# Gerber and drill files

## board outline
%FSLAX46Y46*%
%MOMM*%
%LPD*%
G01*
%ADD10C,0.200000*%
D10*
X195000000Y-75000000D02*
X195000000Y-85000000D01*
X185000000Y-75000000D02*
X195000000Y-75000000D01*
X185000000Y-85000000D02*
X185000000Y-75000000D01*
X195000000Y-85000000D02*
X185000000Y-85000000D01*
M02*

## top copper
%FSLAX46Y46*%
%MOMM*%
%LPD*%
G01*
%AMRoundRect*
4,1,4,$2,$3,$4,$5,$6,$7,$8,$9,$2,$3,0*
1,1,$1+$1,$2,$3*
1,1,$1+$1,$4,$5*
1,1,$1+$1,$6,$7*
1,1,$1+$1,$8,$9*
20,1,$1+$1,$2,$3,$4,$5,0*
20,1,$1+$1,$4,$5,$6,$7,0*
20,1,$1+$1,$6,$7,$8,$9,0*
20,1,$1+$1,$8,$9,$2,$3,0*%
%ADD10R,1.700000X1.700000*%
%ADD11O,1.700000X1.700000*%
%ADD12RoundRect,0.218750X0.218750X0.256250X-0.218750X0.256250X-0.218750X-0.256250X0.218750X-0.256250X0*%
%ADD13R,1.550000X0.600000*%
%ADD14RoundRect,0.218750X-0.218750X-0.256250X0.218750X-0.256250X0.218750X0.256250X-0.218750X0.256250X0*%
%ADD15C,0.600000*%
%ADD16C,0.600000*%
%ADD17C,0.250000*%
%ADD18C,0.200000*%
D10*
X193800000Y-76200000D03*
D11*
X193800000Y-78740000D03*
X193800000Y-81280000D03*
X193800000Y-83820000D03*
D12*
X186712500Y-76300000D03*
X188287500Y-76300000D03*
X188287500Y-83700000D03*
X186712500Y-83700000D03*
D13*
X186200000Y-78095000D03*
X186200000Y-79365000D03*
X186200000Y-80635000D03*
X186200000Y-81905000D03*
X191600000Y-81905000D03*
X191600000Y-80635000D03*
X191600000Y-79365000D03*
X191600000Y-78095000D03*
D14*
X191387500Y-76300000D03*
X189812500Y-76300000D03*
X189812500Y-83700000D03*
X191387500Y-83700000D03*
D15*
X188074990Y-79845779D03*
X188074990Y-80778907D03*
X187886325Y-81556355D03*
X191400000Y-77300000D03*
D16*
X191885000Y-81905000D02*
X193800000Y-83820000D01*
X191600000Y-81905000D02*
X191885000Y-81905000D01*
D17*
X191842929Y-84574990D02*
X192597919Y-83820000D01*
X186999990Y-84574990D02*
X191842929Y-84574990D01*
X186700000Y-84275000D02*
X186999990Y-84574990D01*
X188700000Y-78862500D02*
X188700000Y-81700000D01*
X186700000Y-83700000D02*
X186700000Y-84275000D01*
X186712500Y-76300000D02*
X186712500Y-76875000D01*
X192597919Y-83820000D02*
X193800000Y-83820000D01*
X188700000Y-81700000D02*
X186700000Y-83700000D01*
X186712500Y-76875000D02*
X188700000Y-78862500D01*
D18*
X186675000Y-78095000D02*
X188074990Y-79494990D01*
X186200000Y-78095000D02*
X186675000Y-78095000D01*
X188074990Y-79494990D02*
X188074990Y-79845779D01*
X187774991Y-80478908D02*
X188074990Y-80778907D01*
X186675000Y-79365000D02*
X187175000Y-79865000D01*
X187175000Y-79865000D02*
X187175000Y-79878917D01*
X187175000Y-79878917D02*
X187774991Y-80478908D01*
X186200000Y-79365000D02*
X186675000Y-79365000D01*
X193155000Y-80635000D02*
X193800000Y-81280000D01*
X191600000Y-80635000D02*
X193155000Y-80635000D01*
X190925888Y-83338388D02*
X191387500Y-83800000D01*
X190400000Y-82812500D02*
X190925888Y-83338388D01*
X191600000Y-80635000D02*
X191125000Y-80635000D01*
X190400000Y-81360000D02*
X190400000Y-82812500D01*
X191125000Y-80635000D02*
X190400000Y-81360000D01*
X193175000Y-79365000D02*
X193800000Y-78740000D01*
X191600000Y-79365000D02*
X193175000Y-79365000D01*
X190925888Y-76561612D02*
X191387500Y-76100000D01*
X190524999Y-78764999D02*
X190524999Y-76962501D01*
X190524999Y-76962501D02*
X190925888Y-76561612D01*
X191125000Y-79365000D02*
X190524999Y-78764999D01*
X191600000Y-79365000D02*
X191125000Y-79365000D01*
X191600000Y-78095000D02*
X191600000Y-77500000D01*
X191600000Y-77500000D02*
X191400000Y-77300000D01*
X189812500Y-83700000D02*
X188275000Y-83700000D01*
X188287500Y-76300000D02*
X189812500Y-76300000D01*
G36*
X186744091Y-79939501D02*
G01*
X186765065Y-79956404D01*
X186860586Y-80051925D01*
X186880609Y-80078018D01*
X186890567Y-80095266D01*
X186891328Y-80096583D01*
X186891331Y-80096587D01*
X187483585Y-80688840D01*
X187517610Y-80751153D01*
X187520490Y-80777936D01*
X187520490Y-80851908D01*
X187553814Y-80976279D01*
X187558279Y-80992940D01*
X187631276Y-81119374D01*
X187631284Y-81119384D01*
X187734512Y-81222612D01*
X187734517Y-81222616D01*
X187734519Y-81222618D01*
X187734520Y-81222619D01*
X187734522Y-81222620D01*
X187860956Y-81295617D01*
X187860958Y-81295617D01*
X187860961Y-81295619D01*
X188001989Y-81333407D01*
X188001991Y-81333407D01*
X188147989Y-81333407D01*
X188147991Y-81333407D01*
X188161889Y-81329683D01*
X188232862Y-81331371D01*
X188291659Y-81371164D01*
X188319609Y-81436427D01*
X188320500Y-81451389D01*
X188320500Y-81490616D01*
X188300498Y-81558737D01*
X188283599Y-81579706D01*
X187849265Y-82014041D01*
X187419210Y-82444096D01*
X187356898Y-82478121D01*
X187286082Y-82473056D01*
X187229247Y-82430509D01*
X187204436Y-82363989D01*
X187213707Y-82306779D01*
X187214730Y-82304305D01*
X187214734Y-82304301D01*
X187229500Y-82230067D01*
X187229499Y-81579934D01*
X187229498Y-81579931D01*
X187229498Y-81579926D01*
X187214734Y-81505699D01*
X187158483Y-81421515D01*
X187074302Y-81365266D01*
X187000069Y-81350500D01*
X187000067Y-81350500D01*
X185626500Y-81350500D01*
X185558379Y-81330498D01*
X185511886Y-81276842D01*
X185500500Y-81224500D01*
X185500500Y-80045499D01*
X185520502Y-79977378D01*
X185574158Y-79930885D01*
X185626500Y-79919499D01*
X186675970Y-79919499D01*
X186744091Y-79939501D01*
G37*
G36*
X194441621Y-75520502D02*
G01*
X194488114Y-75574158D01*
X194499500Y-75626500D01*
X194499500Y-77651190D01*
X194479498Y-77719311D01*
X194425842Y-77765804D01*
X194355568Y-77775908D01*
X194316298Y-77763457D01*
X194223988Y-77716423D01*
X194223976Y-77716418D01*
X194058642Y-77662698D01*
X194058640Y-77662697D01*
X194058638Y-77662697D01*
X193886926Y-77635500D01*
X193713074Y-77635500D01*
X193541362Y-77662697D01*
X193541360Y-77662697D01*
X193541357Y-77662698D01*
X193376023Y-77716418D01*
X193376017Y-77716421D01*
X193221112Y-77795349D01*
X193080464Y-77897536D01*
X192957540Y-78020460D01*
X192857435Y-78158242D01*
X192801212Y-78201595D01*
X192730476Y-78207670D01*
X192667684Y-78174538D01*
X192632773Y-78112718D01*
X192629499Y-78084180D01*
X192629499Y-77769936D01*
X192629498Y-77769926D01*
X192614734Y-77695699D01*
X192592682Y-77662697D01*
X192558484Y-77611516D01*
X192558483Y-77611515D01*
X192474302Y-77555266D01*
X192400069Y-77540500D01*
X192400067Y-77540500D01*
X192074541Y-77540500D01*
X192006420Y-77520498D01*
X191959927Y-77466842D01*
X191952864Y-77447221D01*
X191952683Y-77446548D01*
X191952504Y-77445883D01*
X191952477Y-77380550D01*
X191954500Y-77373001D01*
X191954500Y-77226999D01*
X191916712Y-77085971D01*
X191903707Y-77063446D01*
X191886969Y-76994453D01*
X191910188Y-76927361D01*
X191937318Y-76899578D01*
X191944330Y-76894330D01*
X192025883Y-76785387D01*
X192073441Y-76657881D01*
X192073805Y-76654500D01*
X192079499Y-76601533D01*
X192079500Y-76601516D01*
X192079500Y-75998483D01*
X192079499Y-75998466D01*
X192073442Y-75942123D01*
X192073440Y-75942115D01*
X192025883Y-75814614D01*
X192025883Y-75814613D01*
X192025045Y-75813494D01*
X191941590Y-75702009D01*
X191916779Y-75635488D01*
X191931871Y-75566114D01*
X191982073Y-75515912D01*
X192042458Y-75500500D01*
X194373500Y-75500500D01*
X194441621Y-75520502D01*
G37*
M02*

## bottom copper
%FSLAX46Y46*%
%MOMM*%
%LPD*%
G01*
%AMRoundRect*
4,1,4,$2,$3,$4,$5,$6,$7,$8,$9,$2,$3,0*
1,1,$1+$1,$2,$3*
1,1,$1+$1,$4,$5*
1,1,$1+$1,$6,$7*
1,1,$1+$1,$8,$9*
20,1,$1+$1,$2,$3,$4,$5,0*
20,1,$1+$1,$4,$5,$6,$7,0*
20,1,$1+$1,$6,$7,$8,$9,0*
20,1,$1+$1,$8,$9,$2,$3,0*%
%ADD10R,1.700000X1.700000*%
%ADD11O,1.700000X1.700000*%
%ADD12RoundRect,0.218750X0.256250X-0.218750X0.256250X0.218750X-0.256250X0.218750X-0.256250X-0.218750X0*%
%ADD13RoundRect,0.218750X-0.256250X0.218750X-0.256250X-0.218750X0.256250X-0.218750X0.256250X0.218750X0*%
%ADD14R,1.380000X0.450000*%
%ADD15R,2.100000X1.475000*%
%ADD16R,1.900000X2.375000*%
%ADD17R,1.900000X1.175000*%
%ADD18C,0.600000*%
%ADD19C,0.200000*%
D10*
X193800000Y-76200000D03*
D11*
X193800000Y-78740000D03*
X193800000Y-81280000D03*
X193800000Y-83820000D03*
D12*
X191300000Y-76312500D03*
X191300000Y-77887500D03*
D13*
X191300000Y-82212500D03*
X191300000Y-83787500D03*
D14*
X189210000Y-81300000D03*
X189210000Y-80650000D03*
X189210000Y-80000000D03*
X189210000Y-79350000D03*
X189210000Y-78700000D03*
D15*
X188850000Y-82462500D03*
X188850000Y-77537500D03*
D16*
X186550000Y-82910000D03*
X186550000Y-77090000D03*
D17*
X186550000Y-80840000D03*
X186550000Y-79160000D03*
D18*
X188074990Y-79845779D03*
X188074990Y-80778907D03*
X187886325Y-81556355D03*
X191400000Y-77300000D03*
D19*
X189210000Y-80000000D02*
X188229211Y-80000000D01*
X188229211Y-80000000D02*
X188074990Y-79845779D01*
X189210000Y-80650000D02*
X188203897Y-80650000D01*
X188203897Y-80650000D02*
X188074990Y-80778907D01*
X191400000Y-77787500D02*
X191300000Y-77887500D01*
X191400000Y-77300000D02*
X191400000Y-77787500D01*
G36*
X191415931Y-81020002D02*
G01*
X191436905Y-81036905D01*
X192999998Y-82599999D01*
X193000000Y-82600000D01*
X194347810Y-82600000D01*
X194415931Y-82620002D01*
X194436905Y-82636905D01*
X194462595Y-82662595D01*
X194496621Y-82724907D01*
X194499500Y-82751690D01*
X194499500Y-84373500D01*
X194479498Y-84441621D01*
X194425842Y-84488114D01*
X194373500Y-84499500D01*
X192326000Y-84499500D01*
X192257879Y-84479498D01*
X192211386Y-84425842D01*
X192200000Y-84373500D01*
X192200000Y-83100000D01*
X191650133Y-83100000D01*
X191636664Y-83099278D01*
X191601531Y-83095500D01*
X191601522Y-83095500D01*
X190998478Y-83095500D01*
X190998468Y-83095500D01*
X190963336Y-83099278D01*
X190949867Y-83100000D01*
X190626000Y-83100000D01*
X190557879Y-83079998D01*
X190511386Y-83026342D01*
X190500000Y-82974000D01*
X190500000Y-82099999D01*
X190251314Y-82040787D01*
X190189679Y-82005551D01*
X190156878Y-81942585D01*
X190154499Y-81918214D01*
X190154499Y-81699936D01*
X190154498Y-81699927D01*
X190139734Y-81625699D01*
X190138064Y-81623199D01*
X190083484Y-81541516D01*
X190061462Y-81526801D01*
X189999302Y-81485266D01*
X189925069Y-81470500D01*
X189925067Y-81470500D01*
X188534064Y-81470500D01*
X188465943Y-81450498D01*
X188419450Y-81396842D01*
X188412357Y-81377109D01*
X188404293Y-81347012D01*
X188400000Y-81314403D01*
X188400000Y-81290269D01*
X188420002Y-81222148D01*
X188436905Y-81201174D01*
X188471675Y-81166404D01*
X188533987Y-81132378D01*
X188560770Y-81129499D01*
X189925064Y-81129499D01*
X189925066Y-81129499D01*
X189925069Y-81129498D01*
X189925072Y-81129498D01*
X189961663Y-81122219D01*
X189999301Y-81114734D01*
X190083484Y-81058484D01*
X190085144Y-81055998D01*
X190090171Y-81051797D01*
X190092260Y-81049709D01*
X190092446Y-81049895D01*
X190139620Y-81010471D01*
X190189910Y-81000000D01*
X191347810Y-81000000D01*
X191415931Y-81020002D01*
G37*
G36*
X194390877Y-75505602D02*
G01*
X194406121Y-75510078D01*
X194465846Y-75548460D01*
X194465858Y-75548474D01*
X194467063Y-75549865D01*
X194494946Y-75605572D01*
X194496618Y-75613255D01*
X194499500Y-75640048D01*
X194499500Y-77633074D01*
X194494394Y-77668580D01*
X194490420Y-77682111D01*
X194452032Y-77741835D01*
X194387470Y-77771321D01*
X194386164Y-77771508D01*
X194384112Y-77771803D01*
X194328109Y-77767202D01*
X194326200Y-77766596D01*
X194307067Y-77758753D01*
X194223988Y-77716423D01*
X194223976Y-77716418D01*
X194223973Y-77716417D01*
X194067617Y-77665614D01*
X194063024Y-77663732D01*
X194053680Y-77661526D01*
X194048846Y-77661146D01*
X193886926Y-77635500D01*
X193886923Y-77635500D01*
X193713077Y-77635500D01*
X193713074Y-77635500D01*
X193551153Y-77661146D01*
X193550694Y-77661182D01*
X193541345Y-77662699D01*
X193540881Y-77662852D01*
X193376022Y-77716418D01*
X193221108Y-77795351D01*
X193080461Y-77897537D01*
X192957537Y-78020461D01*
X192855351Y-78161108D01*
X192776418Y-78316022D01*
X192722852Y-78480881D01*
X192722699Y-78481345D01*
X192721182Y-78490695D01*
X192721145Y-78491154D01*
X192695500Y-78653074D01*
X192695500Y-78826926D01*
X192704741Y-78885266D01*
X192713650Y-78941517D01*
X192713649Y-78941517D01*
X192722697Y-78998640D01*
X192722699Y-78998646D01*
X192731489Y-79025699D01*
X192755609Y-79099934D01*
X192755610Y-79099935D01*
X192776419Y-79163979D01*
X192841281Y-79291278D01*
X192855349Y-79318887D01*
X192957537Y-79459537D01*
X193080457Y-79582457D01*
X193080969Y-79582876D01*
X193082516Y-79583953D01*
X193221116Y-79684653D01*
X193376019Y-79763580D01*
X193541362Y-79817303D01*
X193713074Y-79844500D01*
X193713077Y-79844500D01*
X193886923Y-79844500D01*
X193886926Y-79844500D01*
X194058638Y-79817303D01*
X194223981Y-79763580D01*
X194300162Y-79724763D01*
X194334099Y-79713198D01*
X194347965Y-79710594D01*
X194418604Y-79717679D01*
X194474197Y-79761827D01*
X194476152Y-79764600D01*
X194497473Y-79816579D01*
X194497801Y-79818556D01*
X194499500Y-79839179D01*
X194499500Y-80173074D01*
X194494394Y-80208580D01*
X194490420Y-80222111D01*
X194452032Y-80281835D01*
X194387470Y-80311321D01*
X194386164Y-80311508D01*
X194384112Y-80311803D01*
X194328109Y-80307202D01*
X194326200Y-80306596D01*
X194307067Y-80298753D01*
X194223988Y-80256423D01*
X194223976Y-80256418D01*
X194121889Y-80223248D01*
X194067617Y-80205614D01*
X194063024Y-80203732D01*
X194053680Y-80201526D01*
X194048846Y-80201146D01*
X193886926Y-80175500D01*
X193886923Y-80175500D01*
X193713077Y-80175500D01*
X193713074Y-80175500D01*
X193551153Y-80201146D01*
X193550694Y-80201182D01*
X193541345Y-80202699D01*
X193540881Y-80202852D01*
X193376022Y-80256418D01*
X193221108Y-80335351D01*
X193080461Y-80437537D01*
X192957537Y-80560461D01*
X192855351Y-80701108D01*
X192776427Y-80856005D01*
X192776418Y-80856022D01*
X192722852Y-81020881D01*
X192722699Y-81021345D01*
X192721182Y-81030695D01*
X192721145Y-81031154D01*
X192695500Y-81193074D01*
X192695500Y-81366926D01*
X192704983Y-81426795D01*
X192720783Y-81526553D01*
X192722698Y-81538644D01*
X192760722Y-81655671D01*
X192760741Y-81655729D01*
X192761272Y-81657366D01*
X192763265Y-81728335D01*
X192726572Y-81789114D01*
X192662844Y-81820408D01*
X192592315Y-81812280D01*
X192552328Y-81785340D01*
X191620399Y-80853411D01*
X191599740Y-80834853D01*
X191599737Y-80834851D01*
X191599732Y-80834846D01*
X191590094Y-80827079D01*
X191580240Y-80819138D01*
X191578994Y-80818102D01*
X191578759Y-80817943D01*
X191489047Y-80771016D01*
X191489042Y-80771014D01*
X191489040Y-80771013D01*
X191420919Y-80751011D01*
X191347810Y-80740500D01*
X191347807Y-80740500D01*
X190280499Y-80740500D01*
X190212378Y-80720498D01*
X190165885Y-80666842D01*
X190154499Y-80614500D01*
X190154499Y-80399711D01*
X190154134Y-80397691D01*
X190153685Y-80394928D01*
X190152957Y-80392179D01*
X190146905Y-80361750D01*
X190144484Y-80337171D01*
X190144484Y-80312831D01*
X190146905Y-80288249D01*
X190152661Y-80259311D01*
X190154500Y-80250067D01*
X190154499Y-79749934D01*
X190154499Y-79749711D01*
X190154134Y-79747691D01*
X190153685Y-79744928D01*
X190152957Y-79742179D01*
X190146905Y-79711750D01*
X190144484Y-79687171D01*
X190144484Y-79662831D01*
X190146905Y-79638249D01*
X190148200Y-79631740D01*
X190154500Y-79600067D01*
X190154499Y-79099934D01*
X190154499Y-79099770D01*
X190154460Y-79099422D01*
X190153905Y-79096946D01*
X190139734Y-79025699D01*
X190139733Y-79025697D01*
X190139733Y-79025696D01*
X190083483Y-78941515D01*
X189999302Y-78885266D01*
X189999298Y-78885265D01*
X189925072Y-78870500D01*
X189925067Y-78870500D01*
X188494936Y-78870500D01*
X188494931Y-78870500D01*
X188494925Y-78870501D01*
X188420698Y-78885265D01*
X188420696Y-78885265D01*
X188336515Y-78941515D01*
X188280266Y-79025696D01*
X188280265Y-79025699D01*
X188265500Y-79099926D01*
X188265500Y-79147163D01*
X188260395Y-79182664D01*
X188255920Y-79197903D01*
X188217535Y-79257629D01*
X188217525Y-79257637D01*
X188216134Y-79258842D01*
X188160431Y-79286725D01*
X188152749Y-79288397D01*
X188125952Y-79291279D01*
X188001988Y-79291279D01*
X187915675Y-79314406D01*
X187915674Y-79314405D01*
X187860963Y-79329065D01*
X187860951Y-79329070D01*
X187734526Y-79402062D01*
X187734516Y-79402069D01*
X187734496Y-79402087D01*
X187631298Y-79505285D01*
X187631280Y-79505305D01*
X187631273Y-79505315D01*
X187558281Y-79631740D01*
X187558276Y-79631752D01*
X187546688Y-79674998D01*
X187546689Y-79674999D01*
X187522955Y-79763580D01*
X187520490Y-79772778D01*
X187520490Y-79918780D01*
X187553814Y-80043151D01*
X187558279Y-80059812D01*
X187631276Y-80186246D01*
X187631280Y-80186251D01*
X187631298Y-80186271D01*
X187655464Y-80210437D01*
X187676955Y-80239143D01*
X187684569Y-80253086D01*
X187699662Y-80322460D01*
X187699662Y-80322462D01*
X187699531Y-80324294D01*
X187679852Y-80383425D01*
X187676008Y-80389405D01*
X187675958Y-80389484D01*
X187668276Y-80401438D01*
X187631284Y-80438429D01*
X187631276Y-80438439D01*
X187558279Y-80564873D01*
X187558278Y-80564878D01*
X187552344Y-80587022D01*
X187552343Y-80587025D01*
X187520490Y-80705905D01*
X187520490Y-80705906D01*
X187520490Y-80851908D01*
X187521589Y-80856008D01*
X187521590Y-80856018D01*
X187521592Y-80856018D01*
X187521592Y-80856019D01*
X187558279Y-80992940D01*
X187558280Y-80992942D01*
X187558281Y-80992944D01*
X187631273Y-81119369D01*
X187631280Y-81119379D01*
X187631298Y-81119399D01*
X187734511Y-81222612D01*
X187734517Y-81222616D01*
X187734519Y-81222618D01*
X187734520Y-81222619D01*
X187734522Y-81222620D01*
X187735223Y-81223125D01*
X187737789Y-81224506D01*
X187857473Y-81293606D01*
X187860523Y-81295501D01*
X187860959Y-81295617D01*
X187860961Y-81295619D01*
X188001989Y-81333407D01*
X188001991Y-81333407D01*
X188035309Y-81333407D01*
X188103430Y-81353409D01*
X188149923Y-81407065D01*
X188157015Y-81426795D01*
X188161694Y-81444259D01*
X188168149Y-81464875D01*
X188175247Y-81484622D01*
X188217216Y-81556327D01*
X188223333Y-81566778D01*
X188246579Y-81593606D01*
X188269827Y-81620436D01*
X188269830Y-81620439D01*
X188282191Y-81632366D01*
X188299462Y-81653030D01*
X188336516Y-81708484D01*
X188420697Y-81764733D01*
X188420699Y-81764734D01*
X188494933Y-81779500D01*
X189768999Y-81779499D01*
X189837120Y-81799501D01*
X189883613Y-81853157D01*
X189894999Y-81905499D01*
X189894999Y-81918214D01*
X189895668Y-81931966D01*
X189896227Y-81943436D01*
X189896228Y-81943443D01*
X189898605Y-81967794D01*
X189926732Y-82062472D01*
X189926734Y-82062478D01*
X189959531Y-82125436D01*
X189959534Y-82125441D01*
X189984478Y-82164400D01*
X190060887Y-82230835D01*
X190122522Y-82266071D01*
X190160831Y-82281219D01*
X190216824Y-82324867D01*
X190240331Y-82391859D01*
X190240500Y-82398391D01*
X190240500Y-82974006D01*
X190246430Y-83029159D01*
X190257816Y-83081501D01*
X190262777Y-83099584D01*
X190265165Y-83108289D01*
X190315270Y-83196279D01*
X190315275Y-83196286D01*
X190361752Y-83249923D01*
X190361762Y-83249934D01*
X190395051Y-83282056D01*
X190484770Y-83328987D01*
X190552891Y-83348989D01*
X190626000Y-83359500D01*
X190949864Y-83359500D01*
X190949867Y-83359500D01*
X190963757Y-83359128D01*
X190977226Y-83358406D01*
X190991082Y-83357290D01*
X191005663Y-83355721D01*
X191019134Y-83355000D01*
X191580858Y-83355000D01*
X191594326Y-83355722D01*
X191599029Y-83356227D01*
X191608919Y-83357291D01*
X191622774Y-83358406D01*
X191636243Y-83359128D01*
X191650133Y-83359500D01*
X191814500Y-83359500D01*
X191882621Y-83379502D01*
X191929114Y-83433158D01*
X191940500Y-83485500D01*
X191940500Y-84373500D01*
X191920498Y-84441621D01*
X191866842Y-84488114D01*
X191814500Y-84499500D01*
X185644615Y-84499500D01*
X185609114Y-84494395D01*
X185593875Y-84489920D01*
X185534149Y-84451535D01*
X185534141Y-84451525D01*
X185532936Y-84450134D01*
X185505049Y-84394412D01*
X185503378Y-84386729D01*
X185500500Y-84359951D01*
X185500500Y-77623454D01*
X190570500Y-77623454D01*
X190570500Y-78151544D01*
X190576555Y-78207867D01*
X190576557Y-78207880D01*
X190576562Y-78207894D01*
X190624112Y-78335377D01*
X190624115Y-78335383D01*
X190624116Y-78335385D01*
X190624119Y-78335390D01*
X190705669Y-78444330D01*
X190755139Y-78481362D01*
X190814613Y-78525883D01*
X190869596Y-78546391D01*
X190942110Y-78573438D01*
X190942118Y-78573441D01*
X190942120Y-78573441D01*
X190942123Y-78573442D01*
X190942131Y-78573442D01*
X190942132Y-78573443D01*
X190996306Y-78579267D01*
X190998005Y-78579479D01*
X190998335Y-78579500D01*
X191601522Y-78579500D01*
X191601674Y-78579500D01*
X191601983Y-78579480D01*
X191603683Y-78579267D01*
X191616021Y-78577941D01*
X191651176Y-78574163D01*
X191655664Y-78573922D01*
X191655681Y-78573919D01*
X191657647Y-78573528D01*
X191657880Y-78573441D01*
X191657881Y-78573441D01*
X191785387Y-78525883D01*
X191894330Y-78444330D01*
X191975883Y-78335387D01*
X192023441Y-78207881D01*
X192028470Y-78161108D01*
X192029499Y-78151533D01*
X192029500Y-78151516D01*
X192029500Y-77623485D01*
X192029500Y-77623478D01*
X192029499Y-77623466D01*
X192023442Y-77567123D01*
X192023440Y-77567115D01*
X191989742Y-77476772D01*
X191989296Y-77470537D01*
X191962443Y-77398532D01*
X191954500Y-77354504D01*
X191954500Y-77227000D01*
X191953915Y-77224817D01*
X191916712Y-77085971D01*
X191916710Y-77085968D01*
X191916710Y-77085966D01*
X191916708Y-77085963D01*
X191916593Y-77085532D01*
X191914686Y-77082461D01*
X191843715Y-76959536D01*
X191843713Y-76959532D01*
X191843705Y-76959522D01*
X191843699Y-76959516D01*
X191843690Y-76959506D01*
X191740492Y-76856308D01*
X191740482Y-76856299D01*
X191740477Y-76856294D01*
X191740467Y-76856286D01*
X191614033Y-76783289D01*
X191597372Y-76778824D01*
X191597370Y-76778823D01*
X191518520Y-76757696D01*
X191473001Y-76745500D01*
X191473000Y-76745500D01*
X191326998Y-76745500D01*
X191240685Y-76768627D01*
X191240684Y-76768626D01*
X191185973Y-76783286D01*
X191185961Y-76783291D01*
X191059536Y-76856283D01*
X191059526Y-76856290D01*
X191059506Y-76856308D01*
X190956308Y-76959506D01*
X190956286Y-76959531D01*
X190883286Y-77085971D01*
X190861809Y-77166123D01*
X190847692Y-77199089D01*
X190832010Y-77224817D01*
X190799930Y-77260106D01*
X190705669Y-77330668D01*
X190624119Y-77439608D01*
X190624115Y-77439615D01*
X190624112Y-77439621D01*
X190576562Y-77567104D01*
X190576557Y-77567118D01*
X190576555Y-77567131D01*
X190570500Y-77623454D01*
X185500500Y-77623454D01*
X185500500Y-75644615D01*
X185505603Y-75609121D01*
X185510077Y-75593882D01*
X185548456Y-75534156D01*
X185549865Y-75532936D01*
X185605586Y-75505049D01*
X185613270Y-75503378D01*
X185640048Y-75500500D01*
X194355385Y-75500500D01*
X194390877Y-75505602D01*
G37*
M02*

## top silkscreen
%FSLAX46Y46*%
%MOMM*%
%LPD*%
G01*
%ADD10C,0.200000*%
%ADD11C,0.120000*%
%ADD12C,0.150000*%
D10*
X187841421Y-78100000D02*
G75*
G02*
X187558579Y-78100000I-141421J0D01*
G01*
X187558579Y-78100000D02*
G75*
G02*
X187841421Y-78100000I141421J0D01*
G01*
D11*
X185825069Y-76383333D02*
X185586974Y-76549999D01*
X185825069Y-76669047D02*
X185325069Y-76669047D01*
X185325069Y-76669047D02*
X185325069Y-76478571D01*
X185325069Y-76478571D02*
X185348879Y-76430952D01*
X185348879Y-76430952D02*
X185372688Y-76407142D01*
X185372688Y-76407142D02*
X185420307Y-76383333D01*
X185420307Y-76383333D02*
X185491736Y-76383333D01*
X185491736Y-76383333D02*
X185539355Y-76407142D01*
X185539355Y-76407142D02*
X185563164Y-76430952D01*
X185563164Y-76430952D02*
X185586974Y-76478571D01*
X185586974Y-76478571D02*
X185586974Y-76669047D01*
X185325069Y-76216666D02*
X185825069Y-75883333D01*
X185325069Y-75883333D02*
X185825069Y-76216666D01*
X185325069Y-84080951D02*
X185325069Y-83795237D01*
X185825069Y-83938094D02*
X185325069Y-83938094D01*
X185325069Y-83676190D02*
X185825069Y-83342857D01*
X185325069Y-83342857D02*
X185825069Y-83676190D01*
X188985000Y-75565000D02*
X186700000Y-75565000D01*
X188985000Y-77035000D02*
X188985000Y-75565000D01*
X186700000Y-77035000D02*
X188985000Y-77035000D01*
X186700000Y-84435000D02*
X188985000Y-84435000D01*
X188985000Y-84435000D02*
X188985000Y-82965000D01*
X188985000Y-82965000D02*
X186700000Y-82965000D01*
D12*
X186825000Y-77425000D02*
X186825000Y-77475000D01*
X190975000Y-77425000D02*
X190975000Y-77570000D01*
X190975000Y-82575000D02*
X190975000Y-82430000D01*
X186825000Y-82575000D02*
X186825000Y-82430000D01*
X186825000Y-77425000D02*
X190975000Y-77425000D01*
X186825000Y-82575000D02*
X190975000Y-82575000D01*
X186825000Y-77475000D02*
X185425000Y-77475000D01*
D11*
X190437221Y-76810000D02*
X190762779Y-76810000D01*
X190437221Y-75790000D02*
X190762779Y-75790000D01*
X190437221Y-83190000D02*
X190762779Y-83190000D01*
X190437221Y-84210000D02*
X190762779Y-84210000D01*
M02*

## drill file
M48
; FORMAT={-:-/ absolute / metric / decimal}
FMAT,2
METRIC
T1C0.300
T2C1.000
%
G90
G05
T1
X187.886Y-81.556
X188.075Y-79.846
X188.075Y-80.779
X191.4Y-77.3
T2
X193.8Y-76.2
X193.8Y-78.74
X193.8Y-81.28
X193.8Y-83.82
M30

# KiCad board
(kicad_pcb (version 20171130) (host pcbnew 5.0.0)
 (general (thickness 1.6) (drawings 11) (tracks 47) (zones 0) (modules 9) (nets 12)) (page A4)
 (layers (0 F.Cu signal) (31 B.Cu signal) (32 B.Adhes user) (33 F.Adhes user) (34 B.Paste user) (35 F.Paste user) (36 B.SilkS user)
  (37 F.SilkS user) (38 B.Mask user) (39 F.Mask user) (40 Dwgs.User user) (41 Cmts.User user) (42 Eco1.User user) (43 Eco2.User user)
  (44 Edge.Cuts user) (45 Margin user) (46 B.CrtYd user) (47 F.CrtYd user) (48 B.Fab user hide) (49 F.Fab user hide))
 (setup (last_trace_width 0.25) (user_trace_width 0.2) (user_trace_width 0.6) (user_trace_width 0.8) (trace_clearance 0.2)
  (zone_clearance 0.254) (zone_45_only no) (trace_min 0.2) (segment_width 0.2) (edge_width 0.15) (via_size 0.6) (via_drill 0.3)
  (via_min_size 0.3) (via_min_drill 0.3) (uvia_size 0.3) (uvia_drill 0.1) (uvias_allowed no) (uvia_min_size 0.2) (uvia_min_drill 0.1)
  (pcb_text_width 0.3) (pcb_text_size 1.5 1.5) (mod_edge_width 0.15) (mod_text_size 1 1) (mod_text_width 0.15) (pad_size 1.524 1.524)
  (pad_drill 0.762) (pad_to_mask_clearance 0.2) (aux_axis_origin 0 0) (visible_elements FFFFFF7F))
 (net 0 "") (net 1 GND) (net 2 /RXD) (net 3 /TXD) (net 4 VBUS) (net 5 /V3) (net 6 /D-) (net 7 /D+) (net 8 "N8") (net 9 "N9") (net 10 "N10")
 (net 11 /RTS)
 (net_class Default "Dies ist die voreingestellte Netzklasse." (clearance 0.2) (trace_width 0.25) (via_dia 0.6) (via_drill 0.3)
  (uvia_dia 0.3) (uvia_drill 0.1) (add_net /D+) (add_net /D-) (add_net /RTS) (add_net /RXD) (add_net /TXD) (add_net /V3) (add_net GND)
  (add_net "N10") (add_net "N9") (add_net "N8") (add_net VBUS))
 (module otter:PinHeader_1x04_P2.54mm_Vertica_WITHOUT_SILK (layer F.Cu) (at 193.8 76.2)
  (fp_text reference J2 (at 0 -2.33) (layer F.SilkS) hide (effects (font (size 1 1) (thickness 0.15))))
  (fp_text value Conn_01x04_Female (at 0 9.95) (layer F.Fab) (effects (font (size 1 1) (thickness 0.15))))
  (pad 1 thru_hole rect (at 0 0) (size 1.7 1.7) (drill 1) (layers *.Cu *.Mask) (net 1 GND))
  (pad 2 thru_hole oval (at 0 2.54) (size 1.7 1.7) (drill 1) (layers *.Cu *.Mask) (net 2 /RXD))
  (pad 3 thru_hole oval (at 0 5.08) (size 1.7 1.7) (drill 1) (layers *.Cu *.Mask) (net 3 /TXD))
  (pad 4 thru_hole oval (at 0 7.62) (size 1.7 1.7) (drill 1) (layers *.Cu *.Mask) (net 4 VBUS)))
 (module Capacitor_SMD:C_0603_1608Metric (layer B.Cu) (at 191.3 77.1 90)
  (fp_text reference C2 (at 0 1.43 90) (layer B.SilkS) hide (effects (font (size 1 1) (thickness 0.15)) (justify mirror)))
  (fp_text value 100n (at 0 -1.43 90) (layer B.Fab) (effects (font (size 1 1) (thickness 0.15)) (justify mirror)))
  (pad 2 smd roundrect (at 0.7875 0 90) (size 0.875 0.95) (layers B.Cu B.Paste B.Mask) (roundrect_rratio 0.25) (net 1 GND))
  (pad 1 smd roundrect (at -0.7875 0 90) (size 0.875 0.95) (layers B.Cu B.Paste B.Mask) (roundrect_rratio 0.25) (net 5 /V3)))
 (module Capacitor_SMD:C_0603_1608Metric (layer B.Cu) (at 191.3 83 270)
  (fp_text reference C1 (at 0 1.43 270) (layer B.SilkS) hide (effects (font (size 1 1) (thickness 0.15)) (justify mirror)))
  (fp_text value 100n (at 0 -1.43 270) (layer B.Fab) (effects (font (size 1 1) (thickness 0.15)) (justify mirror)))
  (pad 1 smd roundrect (at -0.7875 0 270) (size 0.875 0.95) (layers B.Cu B.Paste B.Mask) (roundrect_rratio 0.25) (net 4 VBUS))
  (pad 2 smd roundrect (at 0.7875 0 270) (size 0.875 0.95) (layers B.Cu B.Paste B.Mask) (roundrect_rratio 0.25) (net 1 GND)))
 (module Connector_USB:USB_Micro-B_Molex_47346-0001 (layer B.Cu) (at 187.75 80 90)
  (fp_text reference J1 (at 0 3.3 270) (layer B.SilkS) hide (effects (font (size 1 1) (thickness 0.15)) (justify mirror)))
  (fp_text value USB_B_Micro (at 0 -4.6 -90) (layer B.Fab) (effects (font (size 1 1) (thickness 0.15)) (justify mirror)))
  (pad 1 smd rect (at -1.3 1.46 90) (size 0.45 1.38) (layers B.Cu B.Paste B.Mask) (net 4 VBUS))
  (pad 2 smd rect (at -0.65 1.46 90) (size 0.45 1.38) (layers B.Cu B.Paste B.Mask) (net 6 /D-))
  (pad 3 smd rect (at 0 1.46 90) (size 0.45 1.38) (layers B.Cu B.Paste B.Mask) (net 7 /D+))
  (pad 4 smd rect (at 0.65 1.46 90) (size 0.45 1.38) (layers B.Cu B.Paste B.Mask) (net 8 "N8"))
  (pad 5 smd rect (at 1.3 1.46 90) (size 0.45 1.38) (layers B.Cu B.Paste B.Mask) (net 1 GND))
  (pad 6 smd rect (at -2.4625 1.1 90) (size 1.475 2.1) (layers B.Cu B.Paste B.Mask) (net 1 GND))
  (pad 6 smd rect (at 2.4625 1.1 90) (size 1.475 2.1) (layers B.Cu B.Paste B.Mask) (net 1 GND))
  (pad 6 smd rect (at -2.91 -1.2 90) (size 2.375 1.9) (layers B.Cu B.Paste B.Mask) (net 1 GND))
  (pad 6 smd rect (at 2.91 -1.2 90) (size 2.375 1.9) (layers B.Cu B.Paste B.Mask) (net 1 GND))
  (pad 6 smd rect (at -0.84 -1.2 90) (size 1.175 1.9) (layers B.Cu B.Paste B.Mask) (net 1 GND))
  (pad 6 smd rect (at 0.84 -1.2 90) (size 1.175 1.9) (layers B.Cu B.Paste B.Mask) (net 1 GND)))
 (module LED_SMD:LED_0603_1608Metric (layer F.Cu) (at 187.5 76.3 180)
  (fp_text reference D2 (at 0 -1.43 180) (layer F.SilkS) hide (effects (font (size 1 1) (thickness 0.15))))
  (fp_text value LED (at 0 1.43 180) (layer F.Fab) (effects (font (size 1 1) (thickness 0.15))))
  (fp_line (start -1.485 0.735) (end 0.8 0.735) (layer F.SilkS) (width 0.12))
  (fp_line (start -1.485 -0.735) (end -1.485 0.735) (layer F.SilkS) (width 0.12))
  (fp_line (start 0.8 -0.735) (end -1.485 -0.735) (layer F.SilkS) (width 0.12))
  (pad 2 smd roundrect (at 0.7875 0 180) (size 0.875 0.95) (layers F.Cu F.Paste F.Mask) (roundrect_rratio 0.25) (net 4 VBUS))
  (pad 1 smd roundrect (at -0.7875 0 180) (size 0.875 0.95) (layers F.Cu F.Paste F.Mask) (roundrect_rratio 0.25) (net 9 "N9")))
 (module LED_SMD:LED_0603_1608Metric (layer F.Cu) (at 187.5 83.7 180)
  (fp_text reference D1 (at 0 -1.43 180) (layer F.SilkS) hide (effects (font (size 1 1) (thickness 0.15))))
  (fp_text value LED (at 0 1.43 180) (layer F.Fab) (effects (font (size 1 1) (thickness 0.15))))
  (fp_line (start 0.8 -0.735) (end -1.485 -0.735) (layer F.SilkS) (width 0.12))
  (fp_line (start -1.485 -0.735) (end -1.485 0.735) (layer F.SilkS) (width 0.12))
  (fp_line (start -1.485 0.735) (end 0.8 0.735) (layer F.SilkS) (width 0.12))
  (pad 1 smd roundrect (at -0.7875 0 180) (size 0.875 0.95) (layers F.Cu F.Paste F.Mask) (roundrect_rratio 0.25) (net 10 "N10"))
  (pad 2 smd roundrect (at 0.7875 0 180) (size 0.875 0.95) (layers F.Cu F.Paste F.Mask) (roundrect_rratio 0.25) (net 4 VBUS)))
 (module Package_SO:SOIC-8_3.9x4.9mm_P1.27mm (layer F.Cu) (at 188.9 80)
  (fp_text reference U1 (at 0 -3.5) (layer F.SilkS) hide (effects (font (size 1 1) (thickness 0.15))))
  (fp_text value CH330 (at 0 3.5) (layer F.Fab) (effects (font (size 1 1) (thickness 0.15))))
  (fp_line (start -2.075 -2.575) (end -2.075 -2.525) (layer F.SilkS) (width 0.15))
  (fp_line (start 2.075 -2.575) (end 2.075 -2.43) (layer F.SilkS) (width 0.15))
  (fp_line (start 2.075 2.575) (end 2.075 2.43) (layer F.SilkS) (width 0.15))
  (fp_line (start -2.075 2.575) (end -2.075 2.43) (layer F.SilkS) (width 0.15))
  (fp_line (start -2.075 -2.575) (end 2.075 -2.575) (layer F.SilkS) (width 0.15))
  (fp_line (start -2.075 2.575) (end 2.075 2.575) (layer F.SilkS) (width 0.15))
  (fp_line (start -2.075 -2.525) (end -3.475 -2.525) (layer F.SilkS) (width 0.15))
  (pad 1 smd rect (at -2.7 -1.905) (size 1.55 0.6) (layers F.Cu F.Paste F.Mask) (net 7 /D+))
  (pad 2 smd rect (at -2.7 -0.635) (size 1.55 0.6) (layers F.Cu F.Paste F.Mask) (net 6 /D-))
  (pad 3 smd rect (at -2.7 0.635) (size 1.55 0.6) (layers F.Cu F.Paste F.Mask) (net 1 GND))
  (pad 4 smd rect (at -2.7 1.905) (size 1.55 0.6) (layers F.Cu F.Paste F.Mask) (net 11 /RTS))
  (pad 5 smd rect (at 2.7 1.905) (size 1.55 0.6) (layers F.Cu F.Paste F.Mask) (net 4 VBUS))
  (pad 6 smd rect (at 2.7 0.635) (size 1.55 0.6) (layers F.Cu F.Paste F.Mask) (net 3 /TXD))
  (pad 7 smd rect (at 2.7 -0.635) (size 1.55 0.6) (layers F.Cu F.Paste F.Mask) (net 2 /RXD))
  (pad 8 smd rect (at 2.7 -1.905) (size 1.55 0.6) (layers F.Cu F.Paste F.Mask) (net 5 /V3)))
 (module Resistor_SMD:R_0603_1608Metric (layer F.Cu) (at 190.6 76.3)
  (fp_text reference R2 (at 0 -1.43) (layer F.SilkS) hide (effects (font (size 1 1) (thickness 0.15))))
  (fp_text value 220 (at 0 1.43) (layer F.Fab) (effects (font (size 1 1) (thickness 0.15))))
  (fp_line (start -0.162779 0.51) (end 0.162779 0.51) (layer F.SilkS) (width 0.12))
  (fp_line (start -0.162779 -0.51) (end 0.162779 -0.51) (layer F.SilkS) (width 0.12))
  (pad 2 smd roundrect (at 0.7875 0) (size 0.875 0.95) (layers F.Cu F.Paste F.Mask) (roundrect_rratio 0.25) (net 2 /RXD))
  (pad 1 smd roundrect (at -0.7875 0) (size 0.875 0.95) (layers F.Cu F.Paste F.Mask) (roundrect_rratio 0.25) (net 9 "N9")))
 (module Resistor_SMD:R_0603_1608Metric (layer F.Cu) (at 190.6 83.7)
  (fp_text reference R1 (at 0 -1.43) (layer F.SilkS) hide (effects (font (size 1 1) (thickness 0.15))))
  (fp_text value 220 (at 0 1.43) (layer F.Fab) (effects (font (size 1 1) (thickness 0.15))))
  (fp_line (start -0.162779 -0.51) (end 0.162779 -0.51) (layer F.SilkS) (width 0.12))
  (fp_line (start -0.162779 0.51) (end 0.162779 0.51) (layer F.SilkS) (width 0.12))
  (pad 1 smd roundrect (at -0.7875 0) (size 0.875 0.95) (layers F.Cu F.Paste F.Mask) (roundrect_rratio 0.25) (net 10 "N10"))
  (pad 2 smd roundrect (at 0.7875 0) (size 0.875 0.95) (layers F.Cu F.Paste F.Mask) (roundrect_rratio 0.25) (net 3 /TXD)))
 (gr_circle (center 187.7 78.1) (end 187.8 78.2) (layer F.SilkS) (width 0.2))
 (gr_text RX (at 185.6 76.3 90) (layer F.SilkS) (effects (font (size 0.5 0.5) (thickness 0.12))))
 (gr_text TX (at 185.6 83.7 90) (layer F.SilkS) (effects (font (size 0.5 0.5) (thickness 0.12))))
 (gr_line (start 195 75) (end 195 85) (layer Edge.Cuts) (width 0.2))
 (gr_line (start 185 75) (end 195 75) (layer Edge.Cuts) (width 0.2))
 (gr_line (start 185 85) (end 185 75) (layer Edge.Cuts) (width 0.2))
 (gr_line (start 195 85) (end 185 85) (layer Edge.Cuts) (width 0.2))
 (segment (start 191.885 81.905) (end 193.8 83.82) (width 0.6) (layer F.Cu) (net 4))
 (segment (start 191.6 81.905) (end 191.885 81.905) (width 0.6) (layer F.Cu) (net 4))
 (segment (start 191.842929 84.57499) (end 192.597919 83.82) (width 0.25) (layer F.Cu) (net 4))
 (segment (start 186.99999 84.57499) (end 191.842929 84.57499) (width 0.25) (layer F.Cu) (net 4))
 (segment (start 186.7 84.275) (end 186.99999 84.57499) (width 0.25) (layer F.Cu) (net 4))
 (segment (start 188.7 78.8625) (end 188.7 81.7) (width 0.25) (layer F.Cu) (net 4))
 (segment (start 186.7 83.7) (end 186.7 84.275) (width 0.25) (layer F.Cu) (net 4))
 (segment (start 186.7125 76.3) (end 186.7125 76.875) (width 0.25) (layer F.Cu) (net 4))
 (segment (start 192.597919 83.82) (end 193.8 83.82) (width 0.25) (layer F.Cu) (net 4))
 (segment (start 188.7 81.7) (end 186.7 83.7) (width 0.25) (layer F.Cu) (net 4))
 (segment (start 186.7125 76.875) (end 188.7 78.8625) (width 0.25) (layer F.Cu) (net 4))
 (segment (start 186.675 78.095) (end 188.07499 79.49499) (width 0.2) (layer F.Cu) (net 7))
 (segment (start 189.21 80) (end 188.229211 80) (width 0.2) (layer B.Cu) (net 7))
 (segment (start 188.229211 80) (end 188.07499 79.845779) (width 0.2) (layer B.Cu) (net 7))
 (segment (start 186.2 78.095) (end 186.675 78.095) (width 0.2) (layer F.Cu) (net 7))
 (segment (start 188.07499 79.49499) (end 188.07499 79.845779) (width 0.2) (layer F.Cu) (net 7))
 (via (at 188.07499 79.845779) (size 0.6) (drill 0.3) (layers F.Cu B.Cu) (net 7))
 (segment (start 187.774991 80.478908) (end 188.07499 80.778907) (width 0.2) (layer F.Cu) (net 6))
 (segment (start 189.21 80.65) (end 188.203897 80.65) (width 0.2) (layer B.Cu) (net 6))
 (segment (start 186.675 79.365) (end 187.175 79.865) (width 0.2) (layer F.Cu) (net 6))
 (segment (start 187.175 79.865) (end 187.175 79.878917) (width 0.2) (layer F.Cu) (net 6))
 (segment (start 187.175 79.878917) (end 187.774991 80.478908) (width 0.2) (layer F.Cu) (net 6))
 (segment (start 186.2 79.365) (end 186.675 79.365) (width 0.2) (layer F.Cu) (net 6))
 (segment (start 188.203897 80.65) (end 188.07499 80.778907) (width 0.2) (layer B.Cu) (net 6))
 (via (at 188.07499 80.778907) (size 0.6) (drill 0.3) (layers F.Cu B.Cu) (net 6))
 (via (at 187.886325 81.556355) (size 0.6) (drill 0.3) (layers F.Cu B.Cu) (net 1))
 (segment (start 193.155 80.635) (end 193.8 81.28) (width 0.2) (layer F.Cu) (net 3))
 (segment (start 191.6 80.635) (end 193.155 80.635) (width 0.2) (layer F.Cu) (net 3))
 (segment (start 190.925888 83.338388) (end 191.3875 83.8) (width 0.2) (layer F.Cu) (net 3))
 (segment (start 190.4 82.8125) (end 190.925888 83.338388) (width 0.2) (layer F.Cu) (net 3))
 (segment (start 191.6 80.635) (end 191.125 80.635) (width 0.2) (layer F.Cu) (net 3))
 (segment (start 190.4 81.36) (end 190.4 82.8125) (width 0.2) (layer F.Cu) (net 3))
 (segment (start 191.125 80.635) (end 190.4 81.36) (width 0.2) (layer F.Cu) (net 3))
 (segment (start 193.175 79.365) (end 193.8 78.74) (width 0.2) (layer F.Cu) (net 2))
 (segment (start 191.6 79.365) (end 193.175 79.365) (width 0.2) (layer F.Cu) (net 2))
 (segment (start 190.925888 76.561612) (end 191.3875 76.1) (width 0.2) (layer F.Cu) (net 2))
 (segment (start 190.524999 78.764999) (end 190.524999 76.962501) (width 0.2) (layer F.Cu) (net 2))
 (segment (start 190.524999 76.962501) (end 190.925888 76.561612) (width 0.2) (layer F.Cu) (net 2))
 (segment (start 191.125 79.365) (end 190.524999 78.764999) (width 0.2) (layer F.Cu) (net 2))
 (segment (start 191.6 79.365) (end 191.125 79.365) (width 0.2) (layer F.Cu) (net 2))
 (via (at 191.4 77.3) (size 0.6) (drill 0.3) (layers F.Cu B.Cu) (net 5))
 (segment (start 191.6 78.095) (end 191.6 77.5) (width 0.2) (layer F.Cu) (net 5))
 (segment (start 191.6 77.5) (end 191.4 77.3) (width 0.2) (layer F.Cu) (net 5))
 (segment (start 191.4 77.7875) (end 191.3 77.8875) (width 0.2) (layer B.Cu) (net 5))
 (segment (start 191.4 77.3) (end 191.4 77.7875) (width 0.2) (layer B.Cu) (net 5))
 (segment (start 189.8125 83.7) (end 188.275 83.7) (width 0.2) (layer F.Cu) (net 10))
 (segment (start 188.2875 76.3) (end 189.8125 76.3) (width 0.2) (layer F.Cu) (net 9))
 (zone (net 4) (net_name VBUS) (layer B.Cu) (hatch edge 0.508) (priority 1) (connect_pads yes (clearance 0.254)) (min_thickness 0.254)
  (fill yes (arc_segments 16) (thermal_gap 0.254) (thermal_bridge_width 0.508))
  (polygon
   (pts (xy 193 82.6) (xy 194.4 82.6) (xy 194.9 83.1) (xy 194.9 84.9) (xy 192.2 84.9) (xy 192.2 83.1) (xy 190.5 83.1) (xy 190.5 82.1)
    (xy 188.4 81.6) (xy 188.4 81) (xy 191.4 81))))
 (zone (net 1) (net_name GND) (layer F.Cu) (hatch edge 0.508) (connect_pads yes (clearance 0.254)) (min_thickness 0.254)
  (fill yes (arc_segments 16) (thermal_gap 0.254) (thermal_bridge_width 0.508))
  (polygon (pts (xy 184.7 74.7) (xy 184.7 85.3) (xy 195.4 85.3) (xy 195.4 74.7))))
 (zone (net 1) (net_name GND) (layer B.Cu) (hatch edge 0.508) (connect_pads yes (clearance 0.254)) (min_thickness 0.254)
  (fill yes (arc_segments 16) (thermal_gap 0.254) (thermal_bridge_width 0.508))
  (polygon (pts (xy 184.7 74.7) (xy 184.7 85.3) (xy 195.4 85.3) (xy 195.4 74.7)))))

